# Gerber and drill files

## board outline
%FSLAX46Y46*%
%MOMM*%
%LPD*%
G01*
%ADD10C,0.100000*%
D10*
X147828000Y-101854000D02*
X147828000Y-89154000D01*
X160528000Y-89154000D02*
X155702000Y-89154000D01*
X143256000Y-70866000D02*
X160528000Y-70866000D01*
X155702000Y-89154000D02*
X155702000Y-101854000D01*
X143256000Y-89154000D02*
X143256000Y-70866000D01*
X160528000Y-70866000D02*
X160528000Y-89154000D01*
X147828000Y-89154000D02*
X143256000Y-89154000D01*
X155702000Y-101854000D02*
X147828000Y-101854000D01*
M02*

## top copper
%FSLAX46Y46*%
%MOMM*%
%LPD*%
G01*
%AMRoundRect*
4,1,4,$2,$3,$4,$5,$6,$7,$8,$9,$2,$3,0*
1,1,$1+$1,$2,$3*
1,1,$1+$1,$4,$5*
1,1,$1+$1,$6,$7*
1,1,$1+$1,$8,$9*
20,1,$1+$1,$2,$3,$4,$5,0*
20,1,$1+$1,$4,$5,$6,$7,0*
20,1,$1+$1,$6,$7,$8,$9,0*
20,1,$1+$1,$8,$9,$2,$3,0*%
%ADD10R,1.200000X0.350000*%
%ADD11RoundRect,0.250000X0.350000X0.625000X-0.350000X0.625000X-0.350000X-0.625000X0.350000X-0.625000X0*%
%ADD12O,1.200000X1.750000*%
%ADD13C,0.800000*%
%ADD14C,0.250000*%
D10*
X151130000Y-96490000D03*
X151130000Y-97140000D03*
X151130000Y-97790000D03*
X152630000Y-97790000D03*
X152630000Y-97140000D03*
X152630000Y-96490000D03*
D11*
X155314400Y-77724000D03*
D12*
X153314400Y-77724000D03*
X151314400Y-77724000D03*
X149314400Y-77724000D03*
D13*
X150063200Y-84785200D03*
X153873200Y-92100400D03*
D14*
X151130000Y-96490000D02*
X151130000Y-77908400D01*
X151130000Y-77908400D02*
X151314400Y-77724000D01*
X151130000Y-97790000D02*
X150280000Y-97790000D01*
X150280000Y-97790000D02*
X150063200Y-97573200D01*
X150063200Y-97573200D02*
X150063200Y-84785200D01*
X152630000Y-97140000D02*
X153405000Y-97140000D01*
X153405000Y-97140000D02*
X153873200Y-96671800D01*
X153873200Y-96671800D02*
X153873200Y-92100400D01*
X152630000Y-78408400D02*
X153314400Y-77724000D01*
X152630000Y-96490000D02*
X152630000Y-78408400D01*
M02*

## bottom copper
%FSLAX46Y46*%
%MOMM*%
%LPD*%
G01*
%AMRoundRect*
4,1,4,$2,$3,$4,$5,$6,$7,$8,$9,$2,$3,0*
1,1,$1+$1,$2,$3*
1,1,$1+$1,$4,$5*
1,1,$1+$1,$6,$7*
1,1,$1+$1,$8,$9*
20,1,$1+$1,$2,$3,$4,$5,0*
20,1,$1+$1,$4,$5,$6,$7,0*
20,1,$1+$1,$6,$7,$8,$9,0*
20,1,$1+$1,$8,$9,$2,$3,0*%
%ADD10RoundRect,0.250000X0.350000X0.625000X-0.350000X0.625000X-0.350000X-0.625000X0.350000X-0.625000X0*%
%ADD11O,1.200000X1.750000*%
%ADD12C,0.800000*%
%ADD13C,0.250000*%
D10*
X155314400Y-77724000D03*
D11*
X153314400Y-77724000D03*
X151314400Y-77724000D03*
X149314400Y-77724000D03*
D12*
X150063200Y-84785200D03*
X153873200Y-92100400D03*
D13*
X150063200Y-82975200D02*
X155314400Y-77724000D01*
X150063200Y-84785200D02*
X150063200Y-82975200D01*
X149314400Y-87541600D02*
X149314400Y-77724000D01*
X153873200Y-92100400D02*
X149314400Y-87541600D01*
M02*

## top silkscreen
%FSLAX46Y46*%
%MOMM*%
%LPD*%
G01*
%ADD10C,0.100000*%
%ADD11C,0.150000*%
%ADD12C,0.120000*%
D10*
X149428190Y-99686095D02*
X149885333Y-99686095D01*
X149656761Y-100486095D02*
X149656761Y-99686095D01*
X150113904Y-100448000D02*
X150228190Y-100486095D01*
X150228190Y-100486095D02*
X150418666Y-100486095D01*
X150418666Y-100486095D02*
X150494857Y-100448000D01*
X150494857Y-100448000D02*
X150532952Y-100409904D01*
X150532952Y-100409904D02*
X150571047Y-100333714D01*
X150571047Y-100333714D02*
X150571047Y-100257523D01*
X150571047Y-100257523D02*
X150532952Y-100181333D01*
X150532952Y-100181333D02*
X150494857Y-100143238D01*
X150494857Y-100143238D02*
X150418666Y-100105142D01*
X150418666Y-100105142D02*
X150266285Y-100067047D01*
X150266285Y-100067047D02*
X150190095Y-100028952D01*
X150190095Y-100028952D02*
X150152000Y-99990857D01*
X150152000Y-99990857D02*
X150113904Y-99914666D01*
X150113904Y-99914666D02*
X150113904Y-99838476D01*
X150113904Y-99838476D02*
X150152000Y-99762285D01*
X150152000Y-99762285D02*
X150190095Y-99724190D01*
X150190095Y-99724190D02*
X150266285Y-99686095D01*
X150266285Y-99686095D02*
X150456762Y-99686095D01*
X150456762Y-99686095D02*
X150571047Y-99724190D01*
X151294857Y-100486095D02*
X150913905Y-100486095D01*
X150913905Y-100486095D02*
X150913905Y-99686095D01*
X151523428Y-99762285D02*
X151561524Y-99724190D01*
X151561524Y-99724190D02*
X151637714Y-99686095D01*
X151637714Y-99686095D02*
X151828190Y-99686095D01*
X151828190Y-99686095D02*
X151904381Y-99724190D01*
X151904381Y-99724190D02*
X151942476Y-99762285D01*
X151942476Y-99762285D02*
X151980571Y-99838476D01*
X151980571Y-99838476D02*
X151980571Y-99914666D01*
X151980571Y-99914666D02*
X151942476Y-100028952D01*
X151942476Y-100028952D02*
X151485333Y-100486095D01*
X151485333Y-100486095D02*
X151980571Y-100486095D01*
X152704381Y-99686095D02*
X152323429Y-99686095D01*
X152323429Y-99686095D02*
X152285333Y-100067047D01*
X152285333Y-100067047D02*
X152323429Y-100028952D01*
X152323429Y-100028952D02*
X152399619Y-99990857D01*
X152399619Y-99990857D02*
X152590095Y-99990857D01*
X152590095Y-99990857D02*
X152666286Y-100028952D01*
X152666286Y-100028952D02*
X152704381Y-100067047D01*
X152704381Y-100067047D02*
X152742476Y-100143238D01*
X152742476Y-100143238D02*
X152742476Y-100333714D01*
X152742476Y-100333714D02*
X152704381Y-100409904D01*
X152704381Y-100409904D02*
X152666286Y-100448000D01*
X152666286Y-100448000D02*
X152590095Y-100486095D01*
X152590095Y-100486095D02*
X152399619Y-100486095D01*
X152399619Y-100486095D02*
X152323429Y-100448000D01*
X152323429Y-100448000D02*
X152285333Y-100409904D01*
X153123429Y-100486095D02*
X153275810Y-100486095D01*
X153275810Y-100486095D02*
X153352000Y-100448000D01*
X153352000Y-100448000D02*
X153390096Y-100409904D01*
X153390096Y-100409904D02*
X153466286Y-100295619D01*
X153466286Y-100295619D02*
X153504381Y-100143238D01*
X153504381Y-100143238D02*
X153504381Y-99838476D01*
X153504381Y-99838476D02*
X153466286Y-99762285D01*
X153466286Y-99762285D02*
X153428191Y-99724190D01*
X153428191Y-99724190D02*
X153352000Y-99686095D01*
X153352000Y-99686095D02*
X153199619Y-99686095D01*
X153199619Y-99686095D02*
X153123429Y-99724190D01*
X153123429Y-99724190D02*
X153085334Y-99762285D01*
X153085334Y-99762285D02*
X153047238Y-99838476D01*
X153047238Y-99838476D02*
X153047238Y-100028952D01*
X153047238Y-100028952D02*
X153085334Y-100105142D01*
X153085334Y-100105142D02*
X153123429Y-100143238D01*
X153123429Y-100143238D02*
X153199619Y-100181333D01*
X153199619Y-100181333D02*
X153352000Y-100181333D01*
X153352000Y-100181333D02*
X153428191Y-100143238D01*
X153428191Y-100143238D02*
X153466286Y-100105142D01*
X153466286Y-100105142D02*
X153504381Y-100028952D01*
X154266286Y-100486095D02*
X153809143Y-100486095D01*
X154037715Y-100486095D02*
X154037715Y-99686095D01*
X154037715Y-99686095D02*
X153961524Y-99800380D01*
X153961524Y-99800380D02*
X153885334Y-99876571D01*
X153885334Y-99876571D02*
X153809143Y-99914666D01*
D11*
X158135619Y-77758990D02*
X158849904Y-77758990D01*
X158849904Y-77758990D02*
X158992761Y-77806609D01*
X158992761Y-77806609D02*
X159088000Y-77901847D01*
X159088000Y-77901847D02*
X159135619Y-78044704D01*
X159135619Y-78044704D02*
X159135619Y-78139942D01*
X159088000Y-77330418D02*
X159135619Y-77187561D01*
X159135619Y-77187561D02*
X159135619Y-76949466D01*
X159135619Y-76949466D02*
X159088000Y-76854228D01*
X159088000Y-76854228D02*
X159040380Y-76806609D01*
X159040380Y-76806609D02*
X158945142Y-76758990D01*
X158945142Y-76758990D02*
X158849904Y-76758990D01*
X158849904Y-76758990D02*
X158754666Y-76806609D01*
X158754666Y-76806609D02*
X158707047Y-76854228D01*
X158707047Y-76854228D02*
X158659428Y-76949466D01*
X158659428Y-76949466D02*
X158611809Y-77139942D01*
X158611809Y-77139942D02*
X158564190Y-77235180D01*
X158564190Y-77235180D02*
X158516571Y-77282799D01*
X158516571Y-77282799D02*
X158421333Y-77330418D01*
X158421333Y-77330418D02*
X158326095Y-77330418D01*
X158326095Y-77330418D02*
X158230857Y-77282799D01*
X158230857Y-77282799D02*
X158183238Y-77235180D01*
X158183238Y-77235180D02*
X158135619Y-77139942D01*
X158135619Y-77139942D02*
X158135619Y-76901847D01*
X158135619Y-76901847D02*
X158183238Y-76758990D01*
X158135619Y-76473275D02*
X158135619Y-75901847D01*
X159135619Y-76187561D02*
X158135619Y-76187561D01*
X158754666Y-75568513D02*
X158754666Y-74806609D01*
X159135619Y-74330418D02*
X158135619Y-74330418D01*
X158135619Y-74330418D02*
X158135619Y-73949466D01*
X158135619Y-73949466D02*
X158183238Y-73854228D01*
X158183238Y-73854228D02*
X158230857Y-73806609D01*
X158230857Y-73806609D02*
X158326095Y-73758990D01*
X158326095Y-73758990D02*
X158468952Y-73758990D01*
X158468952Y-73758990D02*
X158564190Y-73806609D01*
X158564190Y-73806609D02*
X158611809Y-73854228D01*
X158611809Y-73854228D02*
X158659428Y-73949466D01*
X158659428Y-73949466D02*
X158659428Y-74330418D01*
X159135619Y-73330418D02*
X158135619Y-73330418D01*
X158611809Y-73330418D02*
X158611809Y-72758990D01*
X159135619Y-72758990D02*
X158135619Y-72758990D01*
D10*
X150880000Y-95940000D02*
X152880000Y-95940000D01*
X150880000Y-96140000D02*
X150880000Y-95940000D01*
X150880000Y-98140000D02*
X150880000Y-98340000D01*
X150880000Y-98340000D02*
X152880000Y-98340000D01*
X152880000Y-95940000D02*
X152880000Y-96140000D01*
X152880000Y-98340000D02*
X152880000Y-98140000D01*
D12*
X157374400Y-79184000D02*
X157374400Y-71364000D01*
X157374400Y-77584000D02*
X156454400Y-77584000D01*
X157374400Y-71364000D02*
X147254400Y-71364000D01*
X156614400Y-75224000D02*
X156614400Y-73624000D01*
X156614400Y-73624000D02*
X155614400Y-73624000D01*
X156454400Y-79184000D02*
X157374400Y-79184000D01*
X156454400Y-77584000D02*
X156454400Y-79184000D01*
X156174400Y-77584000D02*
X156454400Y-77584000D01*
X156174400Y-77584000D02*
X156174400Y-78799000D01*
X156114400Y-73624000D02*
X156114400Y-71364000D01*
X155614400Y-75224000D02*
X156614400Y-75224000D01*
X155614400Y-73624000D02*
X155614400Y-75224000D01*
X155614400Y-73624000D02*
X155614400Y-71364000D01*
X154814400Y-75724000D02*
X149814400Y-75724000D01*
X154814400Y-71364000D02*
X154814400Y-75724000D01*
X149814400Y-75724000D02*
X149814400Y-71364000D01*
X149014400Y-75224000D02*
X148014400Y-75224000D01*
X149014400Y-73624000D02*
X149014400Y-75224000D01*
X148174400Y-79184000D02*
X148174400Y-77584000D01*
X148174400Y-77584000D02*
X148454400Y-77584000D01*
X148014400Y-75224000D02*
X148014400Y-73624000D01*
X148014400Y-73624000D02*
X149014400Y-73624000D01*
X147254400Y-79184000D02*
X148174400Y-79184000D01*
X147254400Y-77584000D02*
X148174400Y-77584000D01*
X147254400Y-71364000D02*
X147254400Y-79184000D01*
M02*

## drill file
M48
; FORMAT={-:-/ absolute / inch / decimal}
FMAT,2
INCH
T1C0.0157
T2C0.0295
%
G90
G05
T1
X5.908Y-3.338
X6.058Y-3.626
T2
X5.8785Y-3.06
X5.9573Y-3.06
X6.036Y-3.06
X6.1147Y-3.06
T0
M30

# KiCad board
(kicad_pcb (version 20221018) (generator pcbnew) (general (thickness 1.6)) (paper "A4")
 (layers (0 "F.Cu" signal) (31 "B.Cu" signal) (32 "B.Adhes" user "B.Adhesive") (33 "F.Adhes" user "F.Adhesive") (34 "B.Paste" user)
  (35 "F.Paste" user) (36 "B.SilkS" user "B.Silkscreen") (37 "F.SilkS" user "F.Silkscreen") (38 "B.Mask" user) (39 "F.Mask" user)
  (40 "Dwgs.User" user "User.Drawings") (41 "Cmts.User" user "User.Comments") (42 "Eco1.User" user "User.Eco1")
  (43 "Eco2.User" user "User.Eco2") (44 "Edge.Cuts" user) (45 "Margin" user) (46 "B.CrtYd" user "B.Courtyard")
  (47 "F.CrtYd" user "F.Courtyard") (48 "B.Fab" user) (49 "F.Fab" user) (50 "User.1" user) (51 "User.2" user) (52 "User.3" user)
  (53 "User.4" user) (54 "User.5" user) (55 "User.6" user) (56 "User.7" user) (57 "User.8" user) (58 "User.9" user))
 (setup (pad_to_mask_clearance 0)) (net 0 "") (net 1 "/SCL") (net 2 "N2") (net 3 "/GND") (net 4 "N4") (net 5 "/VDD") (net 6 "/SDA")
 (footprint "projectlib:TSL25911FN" (layer "F.Cu") (at 151.88 97.14)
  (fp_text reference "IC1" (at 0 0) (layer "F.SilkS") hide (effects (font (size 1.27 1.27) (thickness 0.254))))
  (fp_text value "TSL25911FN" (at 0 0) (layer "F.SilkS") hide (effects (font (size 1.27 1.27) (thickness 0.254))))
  (fp_line (start -1 -1.2) (end 1 -1.2) (stroke (width 0.1) (type solid)) (layer "F.SilkS"))
  (fp_line (start -1 -1) (end -1 -1.2) (stroke (width 0.1) (type solid)) (layer "F.SilkS"))
  (fp_line (start -1 1) (end -1 1.2) (stroke (width 0.1) (type solid)) (layer "F.SilkS"))
  (fp_line (start -1 1.2) (end 1 1.2) (stroke (width 0.1) (type solid)) (layer "F.SilkS"))
  (fp_line (start 1 -1.2) (end 1 -1) (stroke (width 0.1) (type solid)) (layer "F.SilkS"))
  (fp_line (start 1 1.2) (end 1 1) (stroke (width 0.1) (type solid)) (layer "F.SilkS"))
  (pad "1" smd rect (at -0.75 -0.65 90) (size 0.35 1.2) (layers "F.Cu" "F.Paste" "F.Mask") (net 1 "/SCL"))
  (pad "2" smd rect (at -0.75 0 90) (size 0.35 1.2) (layers "F.Cu" "F.Paste" "F.Mask") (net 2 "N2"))
  (pad "3" smd rect (at -0.75 0.65 90) (size 0.35 1.2) (layers "F.Cu" "F.Paste" "F.Mask") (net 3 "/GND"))
  (pad "4" smd rect (at 0.75 0.65 90) (size 0.35 1.2) (layers "F.Cu" "F.Paste" "F.Mask") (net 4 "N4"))
  (pad "5" smd rect (at 0.75 0 90) (size 0.35 1.2) (layers "F.Cu" "F.Paste" "F.Mask") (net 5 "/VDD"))
  (pad "6" smd rect (at 0.75 -0.65 90) (size 0.35 1.2) (layers "F.Cu" "F.Paste" "F.Mask") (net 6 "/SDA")))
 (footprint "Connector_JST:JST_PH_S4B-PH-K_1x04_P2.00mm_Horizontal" (layer "F.Cu") (at 155.3144 77.724 180)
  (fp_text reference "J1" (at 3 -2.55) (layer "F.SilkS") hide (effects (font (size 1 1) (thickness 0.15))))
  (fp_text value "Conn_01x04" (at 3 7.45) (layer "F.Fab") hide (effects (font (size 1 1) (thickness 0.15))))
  (fp_line (start -2.06 -1.46) (end -2.06 6.36) (stroke (width 0.12) (type solid)) (layer "F.SilkS"))
  (fp_line (start -2.06 0.14) (end -1.14 0.14) (stroke (width 0.12) (type solid)) (layer "F.SilkS"))
  (fp_line (start -2.06 6.36) (end 8.06 6.36) (stroke (width 0.12) (type solid)) (layer "F.SilkS"))
  (fp_line (start -1.3 2.5) (end -1.3 4.1) (stroke (width 0.12) (type solid)) (layer "F.SilkS"))
  (fp_line (start -1.3 4.1) (end -0.3 4.1) (stroke (width 0.12) (type solid)) (layer "F.SilkS"))
  (fp_line (start -1.14 -1.46) (end -2.06 -1.46) (stroke (width 0.12) (type solid)) (layer "F.SilkS"))
  (fp_line (start -1.14 0.14) (end -1.14 -1.46) (stroke (width 0.12) (type solid)) (layer "F.SilkS"))
  (fp_line (start -0.86 0.14) (end -1.14 0.14) (stroke (width 0.12) (type solid)) (layer "F.SilkS"))
  (fp_line (start -0.86 0.14) (end -0.86 -1.075) (stroke (width 0.12) (type solid)) (layer "F.SilkS"))
  (fp_line (start -0.8 4.1) (end -0.8 6.36) (stroke (width 0.12) (type solid)) (layer "F.SilkS"))
  (fp_line (start -0.3 2.5) (end -1.3 2.5) (stroke (width 0.12) (type solid)) (layer "F.SilkS"))
  (fp_line (start -0.3 4.1) (end -0.3 2.5) (stroke (width 0.12) (type solid)) (layer "F.SilkS"))
  (fp_line (start -0.3 4.1) (end -0.3 6.36) (stroke (width 0.12) (type solid)) (layer "F.SilkS"))
  (fp_line (start 0.5 2) (end 5.5 2) (stroke (width 0.12) (type solid)) (layer "F.SilkS"))
  (fp_line (start 0.5 6.36) (end 0.5 2) (stroke (width 0.12) (type solid)) (layer "F.SilkS"))
  (fp_line (start 5.5 2) (end 5.5 6.36) (stroke (width 0.12) (type solid)) (layer "F.SilkS"))
  (fp_line (start 6.3 2.5) (end 7.3 2.5) (stroke (width 0.12) (type solid)) (layer "F.SilkS"))
  (fp_line (start 6.3 4.1) (end 6.3 2.5) (stroke (width 0.12) (type solid)) (layer "F.SilkS"))
  (fp_line (start 7.14 -1.46) (end 7.14 0.14) (stroke (width 0.12) (type solid)) (layer "F.SilkS"))
  (fp_line (start 7.14 0.14) (end 6.86 0.14) (stroke (width 0.12) (type solid)) (layer "F.SilkS"))
  (fp_line (start 7.3 2.5) (end 7.3 4.1) (stroke (width 0.12) (type solid)) (layer "F.SilkS"))
  (fp_line (start 7.3 4.1) (end 6.3 4.1) (stroke (width 0.12) (type solid)) (layer "F.SilkS"))
  (fp_line (start 8.06 -1.46) (end 7.14 -1.46) (stroke (width 0.12) (type solid)) (layer "F.SilkS"))
  (fp_line (start 8.06 0.14) (end 7.14 0.14) (stroke (width 0.12) (type solid)) (layer "F.SilkS"))
  (fp_line (start 8.06 6.36) (end 8.06 -1.46) (stroke (width 0.12) (type solid)) (layer "F.SilkS"))
  (pad "1" thru_hole roundrect (at 0 0 180) (size 1.2 1.75) (drill 0.75) (layers "*.Cu" "*.Mask") (roundrect_rratio 0.2083333333)
   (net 3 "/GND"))
  (pad "2" thru_hole oval (at 2 0 180) (size 1.2 1.75) (drill 0.75) (layers "*.Cu" "*.Mask") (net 6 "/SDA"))
  (pad "3" thru_hole oval (at 4 0 180) (size 1.2 1.75) (drill 0.75) (layers "*.Cu" "*.Mask") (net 1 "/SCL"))
  (pad "4" thru_hole oval (at 6 0 180) (size 1.2 1.75) (drill 0.75) (layers "*.Cu" "*.Mask") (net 5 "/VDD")))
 (gr_line (start 147.828 101.854) (end 147.828 89.154) (stroke (width 0.1) (type default)) (layer "Edge.Cuts"))
 (gr_line (start 160.528 89.154) (end 155.702 89.154) (stroke (width 0.1) (type default)) (layer "Edge.Cuts"))
 (gr_line (start 143.256 70.866) (end 160.528 70.866) (stroke (width 0.1) (type default)) (layer "Edge.Cuts"))
 (gr_line (start 155.702 89.154) (end 155.702 101.854) (stroke (width 0.1) (type default)) (layer "Edge.Cuts"))
 (gr_line (start 143.256 89.154) (end 143.256 70.866) (stroke (width 0.1) (type default)) (layer "Edge.Cuts"))
 (gr_line (start 160.528 70.866) (end 160.528 89.154) (stroke (width 0.1) (type default)) (layer "Edge.Cuts"))
 (gr_line (start 147.828 89.154) (end 143.256 89.154) (stroke (width 0.1) (type default)) (layer "Edge.Cuts"))
 (gr_line (start 155.702 101.854) (end 147.828 101.854) (stroke (width 0.1) (type default)) (layer "Edge.Cuts"))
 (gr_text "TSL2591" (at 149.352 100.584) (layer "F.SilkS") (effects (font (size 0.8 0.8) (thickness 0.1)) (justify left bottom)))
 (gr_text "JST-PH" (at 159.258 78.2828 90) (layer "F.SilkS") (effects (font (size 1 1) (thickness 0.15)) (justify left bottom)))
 (segment (start 151.13 96.49) (end 151.13 77.9084) (width 0.25) (layer "F.Cu") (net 1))
 (segment (start 151.13 77.9084) (end 151.3144 77.724) (width 0.25) (layer "F.Cu") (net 1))
 (segment (start 151.13 97.79) (end 150.28 97.79) (width 0.25) (layer "F.Cu") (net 3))
 (segment (start 150.28 97.79) (end 150.0632 97.5732) (width 0.25) (layer "F.Cu") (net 3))
 (segment (start 150.0632 97.5732) (end 150.0632 84.7852) (width 0.25) (layer "F.Cu") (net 3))
 (via (at 150.0632 84.7852) (size 0.8) (drill 0.4) (layers "F.Cu" "B.Cu") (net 3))
 (segment (start 150.0632 82.9752) (end 155.3144 77.724) (width 0.25) (layer "B.Cu") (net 3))
 (segment (start 150.0632 84.7852) (end 150.0632 82.9752) (width 0.25) (layer "B.Cu") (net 3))
 (segment (start 152.63 97.14) (end 153.405 97.14) (width 0.25) (layer "F.Cu") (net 5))
 (segment (start 153.405 97.14) (end 153.8732 96.6718) (width 0.25) (layer "F.Cu") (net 5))
 (segment (start 153.8732 96.6718) (end 153.8732 92.1004) (width 0.25) (layer "F.Cu") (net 5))
 (via (at 153.8732 92.1004) (size 0.8) (drill 0.4) (layers "F.Cu" "B.Cu") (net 5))
 (segment (start 149.3144 87.5416) (end 149.3144 77.724) (width 0.25) (layer "B.Cu") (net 5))
 (segment (start 153.8732 92.1004) (end 149.3144 87.5416) (width 0.25) (layer "B.Cu") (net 5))
 (segment (start 152.63 78.4084) (end 153.3144 77.724) (width 0.25) (layer "F.Cu") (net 6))
 (segment (start 152.63 96.49) (end 152.63 78.4084) (width 0.25) (layer "F.Cu") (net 6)))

